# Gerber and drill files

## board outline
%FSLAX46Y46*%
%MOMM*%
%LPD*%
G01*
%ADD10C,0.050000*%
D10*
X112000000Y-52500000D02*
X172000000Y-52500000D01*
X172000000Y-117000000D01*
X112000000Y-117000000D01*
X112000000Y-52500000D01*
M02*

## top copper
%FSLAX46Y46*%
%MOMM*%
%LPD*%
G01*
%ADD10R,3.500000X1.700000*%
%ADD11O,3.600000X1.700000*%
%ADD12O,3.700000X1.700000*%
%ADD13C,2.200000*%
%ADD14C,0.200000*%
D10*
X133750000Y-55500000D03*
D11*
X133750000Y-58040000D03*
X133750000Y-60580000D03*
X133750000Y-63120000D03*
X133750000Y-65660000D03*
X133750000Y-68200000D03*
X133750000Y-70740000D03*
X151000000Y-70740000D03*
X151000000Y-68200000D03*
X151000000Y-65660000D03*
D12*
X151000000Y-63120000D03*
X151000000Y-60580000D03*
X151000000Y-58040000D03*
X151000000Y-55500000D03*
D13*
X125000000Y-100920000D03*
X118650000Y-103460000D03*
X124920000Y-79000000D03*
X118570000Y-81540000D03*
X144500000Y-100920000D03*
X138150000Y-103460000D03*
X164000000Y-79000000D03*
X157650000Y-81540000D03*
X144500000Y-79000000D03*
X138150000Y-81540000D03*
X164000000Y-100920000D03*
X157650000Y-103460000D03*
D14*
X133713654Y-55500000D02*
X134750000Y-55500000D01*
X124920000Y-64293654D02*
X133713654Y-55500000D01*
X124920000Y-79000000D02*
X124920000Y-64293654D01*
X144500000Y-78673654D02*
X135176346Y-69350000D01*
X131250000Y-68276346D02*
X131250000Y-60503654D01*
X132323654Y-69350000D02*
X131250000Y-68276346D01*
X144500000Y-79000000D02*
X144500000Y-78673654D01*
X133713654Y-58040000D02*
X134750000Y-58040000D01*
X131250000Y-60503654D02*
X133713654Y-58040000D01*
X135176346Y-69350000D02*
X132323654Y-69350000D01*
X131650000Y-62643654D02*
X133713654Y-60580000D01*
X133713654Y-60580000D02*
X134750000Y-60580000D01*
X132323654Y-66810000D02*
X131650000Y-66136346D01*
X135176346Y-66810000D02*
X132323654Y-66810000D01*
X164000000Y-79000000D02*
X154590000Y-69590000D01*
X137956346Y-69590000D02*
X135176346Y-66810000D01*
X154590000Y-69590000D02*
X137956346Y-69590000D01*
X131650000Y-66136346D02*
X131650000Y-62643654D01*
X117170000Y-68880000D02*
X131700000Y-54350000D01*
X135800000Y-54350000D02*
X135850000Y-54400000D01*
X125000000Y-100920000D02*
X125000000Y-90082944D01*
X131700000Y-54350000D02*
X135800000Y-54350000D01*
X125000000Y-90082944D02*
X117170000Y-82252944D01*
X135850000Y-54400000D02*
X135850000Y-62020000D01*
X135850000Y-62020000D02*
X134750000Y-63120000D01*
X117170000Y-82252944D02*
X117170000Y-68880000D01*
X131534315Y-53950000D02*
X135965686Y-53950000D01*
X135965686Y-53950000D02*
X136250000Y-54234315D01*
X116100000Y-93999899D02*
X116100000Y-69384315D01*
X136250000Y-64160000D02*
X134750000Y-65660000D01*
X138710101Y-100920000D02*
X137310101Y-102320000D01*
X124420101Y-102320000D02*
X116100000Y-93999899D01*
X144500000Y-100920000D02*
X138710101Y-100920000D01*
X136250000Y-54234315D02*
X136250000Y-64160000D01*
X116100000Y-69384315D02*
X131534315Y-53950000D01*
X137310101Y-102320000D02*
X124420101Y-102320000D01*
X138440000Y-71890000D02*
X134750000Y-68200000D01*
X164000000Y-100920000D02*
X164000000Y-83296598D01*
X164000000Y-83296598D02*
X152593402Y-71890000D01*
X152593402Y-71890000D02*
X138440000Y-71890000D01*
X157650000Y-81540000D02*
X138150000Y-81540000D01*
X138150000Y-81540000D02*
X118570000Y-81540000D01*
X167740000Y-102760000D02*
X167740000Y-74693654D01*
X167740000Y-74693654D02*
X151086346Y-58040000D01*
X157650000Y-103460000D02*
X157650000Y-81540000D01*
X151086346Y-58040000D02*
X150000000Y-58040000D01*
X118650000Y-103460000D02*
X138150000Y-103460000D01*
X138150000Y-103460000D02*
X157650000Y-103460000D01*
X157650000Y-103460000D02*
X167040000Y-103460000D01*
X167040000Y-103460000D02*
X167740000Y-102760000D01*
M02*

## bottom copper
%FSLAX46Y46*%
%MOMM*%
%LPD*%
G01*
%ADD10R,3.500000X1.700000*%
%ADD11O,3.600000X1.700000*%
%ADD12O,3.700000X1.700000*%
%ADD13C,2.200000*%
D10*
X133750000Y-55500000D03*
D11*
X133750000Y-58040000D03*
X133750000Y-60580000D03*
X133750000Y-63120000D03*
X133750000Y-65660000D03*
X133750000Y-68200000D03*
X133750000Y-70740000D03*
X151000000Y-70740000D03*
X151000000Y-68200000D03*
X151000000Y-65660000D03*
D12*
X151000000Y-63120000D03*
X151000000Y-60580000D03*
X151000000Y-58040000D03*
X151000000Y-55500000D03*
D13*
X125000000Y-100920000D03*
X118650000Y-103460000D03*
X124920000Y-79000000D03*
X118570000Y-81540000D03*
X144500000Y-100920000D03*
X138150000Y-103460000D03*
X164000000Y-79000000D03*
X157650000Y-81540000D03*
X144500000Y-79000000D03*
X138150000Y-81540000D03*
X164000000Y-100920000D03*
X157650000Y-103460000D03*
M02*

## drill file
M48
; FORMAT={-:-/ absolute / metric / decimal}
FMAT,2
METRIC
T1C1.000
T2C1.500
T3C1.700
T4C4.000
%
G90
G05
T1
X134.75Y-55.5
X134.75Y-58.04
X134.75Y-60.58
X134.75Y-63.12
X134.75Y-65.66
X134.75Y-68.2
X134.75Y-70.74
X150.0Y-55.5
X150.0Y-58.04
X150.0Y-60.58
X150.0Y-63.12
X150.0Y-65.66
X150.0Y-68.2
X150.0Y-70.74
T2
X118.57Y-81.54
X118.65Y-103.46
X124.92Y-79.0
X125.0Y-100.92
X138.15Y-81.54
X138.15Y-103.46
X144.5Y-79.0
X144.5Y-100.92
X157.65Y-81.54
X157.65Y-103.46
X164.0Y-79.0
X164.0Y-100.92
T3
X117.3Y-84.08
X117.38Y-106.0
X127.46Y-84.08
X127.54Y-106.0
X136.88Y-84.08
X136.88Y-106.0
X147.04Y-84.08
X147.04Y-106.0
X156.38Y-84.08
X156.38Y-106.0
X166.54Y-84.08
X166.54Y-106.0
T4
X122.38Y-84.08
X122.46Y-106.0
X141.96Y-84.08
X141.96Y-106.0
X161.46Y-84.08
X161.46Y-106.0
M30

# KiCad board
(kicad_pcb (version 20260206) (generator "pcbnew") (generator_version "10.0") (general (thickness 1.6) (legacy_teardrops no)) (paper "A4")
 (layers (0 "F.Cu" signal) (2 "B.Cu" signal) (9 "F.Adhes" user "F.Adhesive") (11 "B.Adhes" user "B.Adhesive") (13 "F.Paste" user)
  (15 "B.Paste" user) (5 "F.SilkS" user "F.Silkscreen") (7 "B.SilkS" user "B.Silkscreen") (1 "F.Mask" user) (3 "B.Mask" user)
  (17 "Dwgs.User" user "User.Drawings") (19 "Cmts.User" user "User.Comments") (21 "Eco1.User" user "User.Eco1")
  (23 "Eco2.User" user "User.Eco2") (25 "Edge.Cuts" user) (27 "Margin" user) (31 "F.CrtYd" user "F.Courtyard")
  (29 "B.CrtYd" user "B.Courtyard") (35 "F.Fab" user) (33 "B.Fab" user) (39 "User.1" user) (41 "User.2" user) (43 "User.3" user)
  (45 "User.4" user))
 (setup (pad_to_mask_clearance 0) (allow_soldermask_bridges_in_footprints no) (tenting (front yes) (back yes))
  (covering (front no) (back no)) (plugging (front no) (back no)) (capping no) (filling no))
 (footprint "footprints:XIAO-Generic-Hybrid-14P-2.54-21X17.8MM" (layer "F.Cu") (at 142.375 63.12)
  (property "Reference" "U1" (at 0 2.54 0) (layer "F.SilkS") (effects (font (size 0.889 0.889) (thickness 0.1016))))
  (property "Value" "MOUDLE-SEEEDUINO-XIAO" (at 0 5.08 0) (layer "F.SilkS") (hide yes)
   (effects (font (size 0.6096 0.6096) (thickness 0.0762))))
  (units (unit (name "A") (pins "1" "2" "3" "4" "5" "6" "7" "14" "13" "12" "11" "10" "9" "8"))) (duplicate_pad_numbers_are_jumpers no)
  (pad "1" thru_hole rect (at -7.625 -7.62) (size 3.5 1.7) (drill 1 (offset -1 0)) (layers "*.Cu" "*.Mask") (remove_unused_layers no)
   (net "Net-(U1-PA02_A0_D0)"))
  (pad "2" thru_hole oval (at -7.625 -5.08) (size 3.6 1.7) (drill 1 (offset -1 0)) (layers "*.Cu" "*.Mask") (remove_unused_layers no)
   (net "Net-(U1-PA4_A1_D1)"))
  (pad "3" thru_hole oval (at -7.625 -2.54) (size 3.6 1.7) (drill 1 (offset -1 0)) (layers "*.Cu" "*.Mask") (remove_unused_layers no)
   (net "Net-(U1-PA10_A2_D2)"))
  (pad "4" thru_hole oval (at -7.625 0) (size 3.6 1.7) (drill 1 (offset -1 0)) (layers "*.Cu" "*.Mask") (remove_unused_layers no)
   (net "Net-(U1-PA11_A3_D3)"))
  (pad "5" thru_hole oval (at -7.625 2.54) (size 3.6 1.7) (drill 1 (offset -1 0)) (layers "*.Cu" "*.Mask") (remove_unused_layers no)
   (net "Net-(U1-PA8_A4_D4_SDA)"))
  (pad "6" thru_hole oval (at -7.625 5.08 180) (size 3.6 1.7) (drill 1 (offset 1 0)) (layers "*.Cu" "*.Mask") (remove_unused_layers no)
   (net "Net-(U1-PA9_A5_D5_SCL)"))
  (pad "7" thru_hole oval (at -7.625 7.62) (size 3.6 1.7) (drill 1 (offset -1 0)) (layers "*.Cu" "*.Mask") (remove_unused_layers no)
   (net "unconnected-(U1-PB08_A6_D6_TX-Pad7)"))
  (pad "8" thru_hole oval (at 7.625 7.62) (size 3.6 1.7) (drill 1 (offset 1 0)) (layers "*.Cu" "*.Mask") (remove_unused_layers no)
   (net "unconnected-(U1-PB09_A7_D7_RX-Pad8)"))
  (pad "9" thru_hole oval (at 7.625 5.08) (size 3.6 1.7) (drill 1 (offset 1 0)) (layers "*.Cu" "*.Mask") (remove_unused_layers no)
   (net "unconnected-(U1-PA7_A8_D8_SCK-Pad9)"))
  (pad "10" thru_hole oval (at 7.625 2.54) (size 3.6 1.7) (drill 1 (offset 1 0)) (layers "*.Cu" "*.Mask") (remove_unused_layers no)
   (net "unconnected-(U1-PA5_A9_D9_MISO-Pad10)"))
  (pad "11" thru_hole oval (at 7.625 0) (size 3.7 1.7) (drill 1 (offset 1 0)) (layers "*.Cu" "*.Mask") (remove_unused_layers no)
   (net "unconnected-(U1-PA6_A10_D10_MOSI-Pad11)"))
  (pad "12" thru_hole oval (at 7.625 -2.54) (size 3.7 1.7) (drill 1 (offset 1 0)) (layers "*.Cu" "*.Mask") (remove_unused_layers no)
   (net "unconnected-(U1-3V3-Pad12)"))
  (pad "13" thru_hole oval (at 7.625 -5.08) (size 3.7 1.7) (drill 1 (offset 1 0)) (layers "*.Cu" "*.Mask") (remove_unused_layers no)
   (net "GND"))
  (pad "14" thru_hole oval (at 7.625 -7.62) (size 3.7 1.7) (drill 1 (offset 1 0)) (layers "*.Cu" "*.Mask") (remove_unused_layers no)
   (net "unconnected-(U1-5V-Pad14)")))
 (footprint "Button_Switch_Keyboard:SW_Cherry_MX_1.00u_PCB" (layer "F.Cu") (at 125 100.92)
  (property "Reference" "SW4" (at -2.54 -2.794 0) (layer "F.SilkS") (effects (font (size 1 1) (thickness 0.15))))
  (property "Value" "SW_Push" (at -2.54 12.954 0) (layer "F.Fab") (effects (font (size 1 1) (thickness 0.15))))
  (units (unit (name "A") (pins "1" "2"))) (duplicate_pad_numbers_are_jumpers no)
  (pad "" np_thru_hole circle (at -7.62 5.08) (size 1.7 1.7) (drill 1.7) (layers "*.Cu" "*.Mask"))
  (pad "" np_thru_hole circle (at -2.54 5.08) (size 4 4) (drill 4) (layers "*.Cu" "*.Mask"))
  (pad "" np_thru_hole circle (at 2.54 5.08) (size 1.7 1.7) (drill 1.7) (layers "*.Cu" "*.Mask"))
  (pad "1" thru_hole circle (at 0 0) (size 2.2 2.2) (drill 1.5) (layers "*.Cu" "*.Mask") (remove_unused_layers no)
   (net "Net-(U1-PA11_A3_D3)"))
  (pad "2" thru_hole circle (at -6.35 2.54) (size 2.2 2.2) (drill 1.5) (layers "*.Cu" "*.Mask") (remove_unused_layers no) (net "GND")))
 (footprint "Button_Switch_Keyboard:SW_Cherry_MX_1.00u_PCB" (layer "F.Cu") (at 124.92 79)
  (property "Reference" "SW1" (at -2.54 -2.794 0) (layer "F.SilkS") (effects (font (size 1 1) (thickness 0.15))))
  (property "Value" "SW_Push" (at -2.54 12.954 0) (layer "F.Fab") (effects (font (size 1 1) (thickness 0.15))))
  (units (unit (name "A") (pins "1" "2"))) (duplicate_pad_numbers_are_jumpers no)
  (pad "" np_thru_hole circle (at -7.62 5.08) (size 1.7 1.7) (drill 1.7) (layers "*.Cu" "*.Mask"))
  (pad "" np_thru_hole circle (at -2.54 5.08) (size 4 4) (drill 4) (layers "*.Cu" "*.Mask"))
  (pad "" np_thru_hole circle (at 2.54 5.08) (size 1.7 1.7) (drill 1.7) (layers "*.Cu" "*.Mask"))
  (pad "1" thru_hole circle (at 0 0) (size 2.2 2.2) (drill 1.5) (layers "*.Cu" "*.Mask") (remove_unused_layers no)
   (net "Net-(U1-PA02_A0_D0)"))
  (pad "2" thru_hole circle (at -6.35 2.54) (size 2.2 2.2) (drill 1.5) (layers "*.Cu" "*.Mask") (remove_unused_layers no) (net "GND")))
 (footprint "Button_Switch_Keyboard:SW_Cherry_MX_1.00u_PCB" (layer "F.Cu") (at 144.5 100.92)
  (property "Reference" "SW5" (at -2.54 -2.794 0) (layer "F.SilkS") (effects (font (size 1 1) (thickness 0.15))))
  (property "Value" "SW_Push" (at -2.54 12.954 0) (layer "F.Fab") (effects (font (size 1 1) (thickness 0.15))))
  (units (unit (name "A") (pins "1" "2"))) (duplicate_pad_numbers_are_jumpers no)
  (pad "" np_thru_hole circle (at -7.62 5.08) (size 1.7 1.7) (drill 1.7) (layers "*.Cu" "*.Mask"))
  (pad "" np_thru_hole circle (at -2.54 5.08) (size 4 4) (drill 4) (layers "*.Cu" "*.Mask"))
  (pad "" np_thru_hole circle (at 2.54 5.08) (size 1.7 1.7) (drill 1.7) (layers "*.Cu" "*.Mask"))
  (pad "1" thru_hole circle (at 0 0) (size 2.2 2.2) (drill 1.5) (layers "*.Cu" "*.Mask") (remove_unused_layers no)
   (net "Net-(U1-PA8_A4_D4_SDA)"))
  (pad "2" thru_hole circle (at -6.35 2.54) (size 2.2 2.2) (drill 1.5) (layers "*.Cu" "*.Mask") (remove_unused_layers no) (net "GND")))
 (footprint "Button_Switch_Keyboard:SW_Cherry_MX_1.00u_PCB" (layer "F.Cu") (at 164 79)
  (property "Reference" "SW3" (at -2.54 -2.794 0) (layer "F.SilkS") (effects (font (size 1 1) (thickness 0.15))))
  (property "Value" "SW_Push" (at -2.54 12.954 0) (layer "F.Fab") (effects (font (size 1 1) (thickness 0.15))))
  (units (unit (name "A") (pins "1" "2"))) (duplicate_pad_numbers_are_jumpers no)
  (pad "" np_thru_hole circle (at -7.62 5.08) (size 1.7 1.7) (drill 1.7) (layers "*.Cu" "*.Mask"))
  (pad "" np_thru_hole circle (at -2.54 5.08) (size 4 4) (drill 4) (layers "*.Cu" "*.Mask"))
  (pad "" np_thru_hole circle (at 2.54 5.08) (size 1.7 1.7) (drill 1.7) (layers "*.Cu" "*.Mask"))
  (pad "1" thru_hole circle (at 0 0) (size 2.2 2.2) (drill 1.5) (layers "*.Cu" "*.Mask") (remove_unused_layers no)
   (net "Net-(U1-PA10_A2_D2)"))
  (pad "2" thru_hole circle (at -6.35 2.54) (size 2.2 2.2) (drill 1.5) (layers "*.Cu" "*.Mask") (remove_unused_layers no) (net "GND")))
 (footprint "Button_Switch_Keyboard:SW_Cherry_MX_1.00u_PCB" (layer "F.Cu") (at 144.5 79)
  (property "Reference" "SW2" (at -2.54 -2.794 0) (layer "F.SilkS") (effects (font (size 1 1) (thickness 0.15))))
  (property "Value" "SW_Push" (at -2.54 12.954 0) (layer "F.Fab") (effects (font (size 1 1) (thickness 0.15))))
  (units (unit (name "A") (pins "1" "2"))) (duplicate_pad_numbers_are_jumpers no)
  (pad "" np_thru_hole circle (at -7.62 5.08) (size 1.7 1.7) (drill 1.7) (layers "*.Cu" "*.Mask"))
  (pad "" np_thru_hole circle (at -2.54 5.08) (size 4 4) (drill 4) (layers "*.Cu" "*.Mask"))
  (pad "" np_thru_hole circle (at 2.54 5.08) (size 1.7 1.7) (drill 1.7) (layers "*.Cu" "*.Mask"))
  (pad "1" thru_hole circle (at 0 0) (size 2.2 2.2) (drill 1.5) (layers "*.Cu" "*.Mask") (remove_unused_layers no)
   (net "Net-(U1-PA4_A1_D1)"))
  (pad "2" thru_hole circle (at -6.35 2.54) (size 2.2 2.2) (drill 1.5) (layers "*.Cu" "*.Mask") (remove_unused_layers no) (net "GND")))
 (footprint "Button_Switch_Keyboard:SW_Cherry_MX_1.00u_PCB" (layer "F.Cu") (at 164 100.92)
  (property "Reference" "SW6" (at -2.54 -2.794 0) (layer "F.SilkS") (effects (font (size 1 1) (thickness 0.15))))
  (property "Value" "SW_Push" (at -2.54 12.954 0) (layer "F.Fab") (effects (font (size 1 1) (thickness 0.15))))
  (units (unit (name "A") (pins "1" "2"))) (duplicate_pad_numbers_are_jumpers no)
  (pad "" np_thru_hole circle (at -7.62 5.08) (size 1.7 1.7) (drill 1.7) (layers "*.Cu" "*.Mask"))
  (pad "" np_thru_hole circle (at -2.54 5.08) (size 4 4) (drill 4) (layers "*.Cu" "*.Mask"))
  (pad "" np_thru_hole circle (at 2.54 5.08) (size 1.7 1.7) (drill 1.7) (layers "*.Cu" "*.Mask"))
  (pad "1" thru_hole circle (at 0 0) (size 2.2 2.2) (drill 1.5) (layers "*.Cu" "*.Mask") (remove_unused_layers no)
   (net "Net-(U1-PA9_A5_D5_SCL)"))
  (pad "2" thru_hole circle (at -6.35 2.54) (size 2.2 2.2) (drill 1.5) (layers "*.Cu" "*.Mask") (remove_unused_layers no) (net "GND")))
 (gr_rect (start 112 52.5) (end 172 117) (stroke (width 0.05) (type default)) (fill no) (layer "Edge.Cuts"))
 (segment (start 133.713654 55.5) (end 134.75 55.5) (width 0.2) (layer "F.Cu") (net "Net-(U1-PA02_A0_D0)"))
 (segment (start 124.92 64.293654) (end 133.713654 55.5) (width 0.2) (layer "F.Cu") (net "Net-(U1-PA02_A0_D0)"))
 (segment (start 124.92 79) (end 124.92 64.293654) (width 0.2) (layer "F.Cu") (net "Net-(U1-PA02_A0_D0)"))
 (segment (start 144.5 78.673654) (end 135.176346 69.35) (width 0.2) (layer "F.Cu") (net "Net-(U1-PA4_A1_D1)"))
 (segment (start 131.25 68.276346) (end 131.25 60.503654) (width 0.2) (layer "F.Cu") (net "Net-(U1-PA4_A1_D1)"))
 (segment (start 132.323654 69.35) (end 131.25 68.276346) (width 0.2) (layer "F.Cu") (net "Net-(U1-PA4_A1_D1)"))
 (segment (start 144.5 79) (end 144.5 78.673654) (width 0.2) (layer "F.Cu") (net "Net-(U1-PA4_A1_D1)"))
 (segment (start 133.713654 58.04) (end 134.75 58.04) (width 0.2) (layer "F.Cu") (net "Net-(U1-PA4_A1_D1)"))
 (segment (start 131.25 60.503654) (end 133.713654 58.04) (width 0.2) (layer "F.Cu") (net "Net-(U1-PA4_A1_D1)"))
 (segment (start 135.176346 69.35) (end 132.323654 69.35) (width 0.2) (layer "F.Cu") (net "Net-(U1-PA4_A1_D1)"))
 (segment (start 131.65 62.643654) (end 133.713654 60.58) (width 0.2) (layer "F.Cu") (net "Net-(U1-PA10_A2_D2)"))
 (segment (start 133.713654 60.58) (end 134.75 60.58) (width 0.2) (layer "F.Cu") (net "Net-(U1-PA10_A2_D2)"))
 (segment (start 132.323654 66.81) (end 131.65 66.136346) (width 0.2) (layer "F.Cu") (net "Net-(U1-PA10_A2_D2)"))
 (segment (start 135.176346 66.81) (end 132.323654 66.81) (width 0.2) (layer "F.Cu") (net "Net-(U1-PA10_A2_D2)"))
 (segment (start 164 79) (end 154.59 69.59) (width 0.2) (layer "F.Cu") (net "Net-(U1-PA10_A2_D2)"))
 (segment (start 137.956346 69.59) (end 135.176346 66.81) (width 0.2) (layer "F.Cu") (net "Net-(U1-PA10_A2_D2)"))
 (segment (start 154.59 69.59) (end 137.956346 69.59) (width 0.2) (layer "F.Cu") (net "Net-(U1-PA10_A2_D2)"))
 (segment (start 131.65 66.136346) (end 131.65 62.643654) (width 0.2) (layer "F.Cu") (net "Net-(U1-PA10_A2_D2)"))
 (segment (start 117.17 68.88) (end 131.7 54.35) (width 0.2) (layer "F.Cu") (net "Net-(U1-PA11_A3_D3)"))
 (segment (start 135.8 54.35) (end 135.85 54.4) (width 0.2) (layer "F.Cu") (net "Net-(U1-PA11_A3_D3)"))
 (segment (start 125 100.92) (end 125 90.082944) (width 0.2) (layer "F.Cu") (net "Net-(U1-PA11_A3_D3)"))
 (segment (start 131.7 54.35) (end 135.8 54.35) (width 0.2) (layer "F.Cu") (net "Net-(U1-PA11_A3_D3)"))
 (segment (start 125 90.082944) (end 117.17 82.252944) (width 0.2) (layer "F.Cu") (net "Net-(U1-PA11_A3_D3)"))
 (segment (start 135.85 54.4) (end 135.85 62.02) (width 0.2) (layer "F.Cu") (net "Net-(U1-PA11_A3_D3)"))
 (segment (start 135.85 62.02) (end 134.75 63.12) (width 0.2) (layer "F.Cu") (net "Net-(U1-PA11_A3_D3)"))
 (segment (start 117.17 82.252944) (end 117.17 68.88) (width 0.2) (layer "F.Cu") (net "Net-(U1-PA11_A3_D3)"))
 (segment (start 131.534315 53.95) (end 135.965686 53.95) (width 0.2) (layer "F.Cu") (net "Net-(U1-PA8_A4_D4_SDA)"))
 (segment (start 135.965686 53.95) (end 136.25 54.234315) (width 0.2) (layer "F.Cu") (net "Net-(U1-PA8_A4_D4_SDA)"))
 (segment (start 116.1 93.999899) (end 116.1 69.384315) (width 0.2) (layer "F.Cu") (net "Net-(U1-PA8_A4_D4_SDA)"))
 (segment (start 136.25 64.16) (end 134.75 65.66) (width 0.2) (layer "F.Cu") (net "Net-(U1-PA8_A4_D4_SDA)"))
 (segment (start 138.710101 100.92) (end 137.310101 102.32) (width 0.2) (layer "F.Cu") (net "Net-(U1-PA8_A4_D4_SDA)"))
 (segment (start 124.420101 102.32) (end 116.1 93.999899) (width 0.2) (layer "F.Cu") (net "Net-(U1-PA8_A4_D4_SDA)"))
 (segment (start 144.5 100.92) (end 138.710101 100.92) (width 0.2) (layer "F.Cu") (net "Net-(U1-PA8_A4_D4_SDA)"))
 (segment (start 136.25 54.234315) (end 136.25 64.16) (width 0.2) (layer "F.Cu") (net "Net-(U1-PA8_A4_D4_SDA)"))
 (segment (start 116.1 69.384315) (end 131.534315 53.95) (width 0.2) (layer "F.Cu") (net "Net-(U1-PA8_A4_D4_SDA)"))
 (segment (start 137.310101 102.32) (end 124.420101 102.32) (width 0.2) (layer "F.Cu") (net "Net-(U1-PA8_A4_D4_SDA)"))
 (segment (start 138.44 71.89) (end 134.75 68.2) (width 0.2) (layer "F.Cu") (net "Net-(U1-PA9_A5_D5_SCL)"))
 (segment (start 164 100.92) (end 164 83.296598) (width 0.2) (layer "F.Cu") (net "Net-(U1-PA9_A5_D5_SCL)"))
 (segment (start 164 83.296598) (end 152.593402 71.89) (width 0.2) (layer "F.Cu") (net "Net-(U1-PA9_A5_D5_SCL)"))
 (segment (start 152.593402 71.89) (end 138.44 71.89) (width 0.2) (layer "F.Cu") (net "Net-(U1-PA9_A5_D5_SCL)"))
 (segment (start 157.65 81.54) (end 138.15 81.54) (width 0.2) (layer "F.Cu") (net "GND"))
 (segment (start 138.15 81.54) (end 118.57 81.54) (width 0.2) (layer "F.Cu") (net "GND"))
 (segment (start 167.74 102.76) (end 167.74 74.693654) (width 0.2) (layer "F.Cu") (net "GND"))
 (segment (start 167.74 74.693654) (end 151.086346 58.04) (width 0.2) (layer "F.Cu") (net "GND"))
 (segment (start 157.65 103.46) (end 157.65 81.54) (width 0.2) (layer "F.Cu") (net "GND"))
 (segment (start 151.086346 58.04) (end 150 58.04) (width 0.2) (layer "F.Cu") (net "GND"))
 (segment (start 118.65 103.46) (end 138.15 103.46) (width 0.2) (layer "F.Cu") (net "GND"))
 (segment (start 138.15 103.46) (end 157.65 103.46) (width 0.2) (layer "F.Cu") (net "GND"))
 (segment (start 157.65 103.46) (end 167.04 103.46) (width 0.2) (layer "F.Cu") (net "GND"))
 (segment (start 167.04 103.46) (end 167.74 102.76) (width 0.2) (layer "F.Cu") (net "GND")))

